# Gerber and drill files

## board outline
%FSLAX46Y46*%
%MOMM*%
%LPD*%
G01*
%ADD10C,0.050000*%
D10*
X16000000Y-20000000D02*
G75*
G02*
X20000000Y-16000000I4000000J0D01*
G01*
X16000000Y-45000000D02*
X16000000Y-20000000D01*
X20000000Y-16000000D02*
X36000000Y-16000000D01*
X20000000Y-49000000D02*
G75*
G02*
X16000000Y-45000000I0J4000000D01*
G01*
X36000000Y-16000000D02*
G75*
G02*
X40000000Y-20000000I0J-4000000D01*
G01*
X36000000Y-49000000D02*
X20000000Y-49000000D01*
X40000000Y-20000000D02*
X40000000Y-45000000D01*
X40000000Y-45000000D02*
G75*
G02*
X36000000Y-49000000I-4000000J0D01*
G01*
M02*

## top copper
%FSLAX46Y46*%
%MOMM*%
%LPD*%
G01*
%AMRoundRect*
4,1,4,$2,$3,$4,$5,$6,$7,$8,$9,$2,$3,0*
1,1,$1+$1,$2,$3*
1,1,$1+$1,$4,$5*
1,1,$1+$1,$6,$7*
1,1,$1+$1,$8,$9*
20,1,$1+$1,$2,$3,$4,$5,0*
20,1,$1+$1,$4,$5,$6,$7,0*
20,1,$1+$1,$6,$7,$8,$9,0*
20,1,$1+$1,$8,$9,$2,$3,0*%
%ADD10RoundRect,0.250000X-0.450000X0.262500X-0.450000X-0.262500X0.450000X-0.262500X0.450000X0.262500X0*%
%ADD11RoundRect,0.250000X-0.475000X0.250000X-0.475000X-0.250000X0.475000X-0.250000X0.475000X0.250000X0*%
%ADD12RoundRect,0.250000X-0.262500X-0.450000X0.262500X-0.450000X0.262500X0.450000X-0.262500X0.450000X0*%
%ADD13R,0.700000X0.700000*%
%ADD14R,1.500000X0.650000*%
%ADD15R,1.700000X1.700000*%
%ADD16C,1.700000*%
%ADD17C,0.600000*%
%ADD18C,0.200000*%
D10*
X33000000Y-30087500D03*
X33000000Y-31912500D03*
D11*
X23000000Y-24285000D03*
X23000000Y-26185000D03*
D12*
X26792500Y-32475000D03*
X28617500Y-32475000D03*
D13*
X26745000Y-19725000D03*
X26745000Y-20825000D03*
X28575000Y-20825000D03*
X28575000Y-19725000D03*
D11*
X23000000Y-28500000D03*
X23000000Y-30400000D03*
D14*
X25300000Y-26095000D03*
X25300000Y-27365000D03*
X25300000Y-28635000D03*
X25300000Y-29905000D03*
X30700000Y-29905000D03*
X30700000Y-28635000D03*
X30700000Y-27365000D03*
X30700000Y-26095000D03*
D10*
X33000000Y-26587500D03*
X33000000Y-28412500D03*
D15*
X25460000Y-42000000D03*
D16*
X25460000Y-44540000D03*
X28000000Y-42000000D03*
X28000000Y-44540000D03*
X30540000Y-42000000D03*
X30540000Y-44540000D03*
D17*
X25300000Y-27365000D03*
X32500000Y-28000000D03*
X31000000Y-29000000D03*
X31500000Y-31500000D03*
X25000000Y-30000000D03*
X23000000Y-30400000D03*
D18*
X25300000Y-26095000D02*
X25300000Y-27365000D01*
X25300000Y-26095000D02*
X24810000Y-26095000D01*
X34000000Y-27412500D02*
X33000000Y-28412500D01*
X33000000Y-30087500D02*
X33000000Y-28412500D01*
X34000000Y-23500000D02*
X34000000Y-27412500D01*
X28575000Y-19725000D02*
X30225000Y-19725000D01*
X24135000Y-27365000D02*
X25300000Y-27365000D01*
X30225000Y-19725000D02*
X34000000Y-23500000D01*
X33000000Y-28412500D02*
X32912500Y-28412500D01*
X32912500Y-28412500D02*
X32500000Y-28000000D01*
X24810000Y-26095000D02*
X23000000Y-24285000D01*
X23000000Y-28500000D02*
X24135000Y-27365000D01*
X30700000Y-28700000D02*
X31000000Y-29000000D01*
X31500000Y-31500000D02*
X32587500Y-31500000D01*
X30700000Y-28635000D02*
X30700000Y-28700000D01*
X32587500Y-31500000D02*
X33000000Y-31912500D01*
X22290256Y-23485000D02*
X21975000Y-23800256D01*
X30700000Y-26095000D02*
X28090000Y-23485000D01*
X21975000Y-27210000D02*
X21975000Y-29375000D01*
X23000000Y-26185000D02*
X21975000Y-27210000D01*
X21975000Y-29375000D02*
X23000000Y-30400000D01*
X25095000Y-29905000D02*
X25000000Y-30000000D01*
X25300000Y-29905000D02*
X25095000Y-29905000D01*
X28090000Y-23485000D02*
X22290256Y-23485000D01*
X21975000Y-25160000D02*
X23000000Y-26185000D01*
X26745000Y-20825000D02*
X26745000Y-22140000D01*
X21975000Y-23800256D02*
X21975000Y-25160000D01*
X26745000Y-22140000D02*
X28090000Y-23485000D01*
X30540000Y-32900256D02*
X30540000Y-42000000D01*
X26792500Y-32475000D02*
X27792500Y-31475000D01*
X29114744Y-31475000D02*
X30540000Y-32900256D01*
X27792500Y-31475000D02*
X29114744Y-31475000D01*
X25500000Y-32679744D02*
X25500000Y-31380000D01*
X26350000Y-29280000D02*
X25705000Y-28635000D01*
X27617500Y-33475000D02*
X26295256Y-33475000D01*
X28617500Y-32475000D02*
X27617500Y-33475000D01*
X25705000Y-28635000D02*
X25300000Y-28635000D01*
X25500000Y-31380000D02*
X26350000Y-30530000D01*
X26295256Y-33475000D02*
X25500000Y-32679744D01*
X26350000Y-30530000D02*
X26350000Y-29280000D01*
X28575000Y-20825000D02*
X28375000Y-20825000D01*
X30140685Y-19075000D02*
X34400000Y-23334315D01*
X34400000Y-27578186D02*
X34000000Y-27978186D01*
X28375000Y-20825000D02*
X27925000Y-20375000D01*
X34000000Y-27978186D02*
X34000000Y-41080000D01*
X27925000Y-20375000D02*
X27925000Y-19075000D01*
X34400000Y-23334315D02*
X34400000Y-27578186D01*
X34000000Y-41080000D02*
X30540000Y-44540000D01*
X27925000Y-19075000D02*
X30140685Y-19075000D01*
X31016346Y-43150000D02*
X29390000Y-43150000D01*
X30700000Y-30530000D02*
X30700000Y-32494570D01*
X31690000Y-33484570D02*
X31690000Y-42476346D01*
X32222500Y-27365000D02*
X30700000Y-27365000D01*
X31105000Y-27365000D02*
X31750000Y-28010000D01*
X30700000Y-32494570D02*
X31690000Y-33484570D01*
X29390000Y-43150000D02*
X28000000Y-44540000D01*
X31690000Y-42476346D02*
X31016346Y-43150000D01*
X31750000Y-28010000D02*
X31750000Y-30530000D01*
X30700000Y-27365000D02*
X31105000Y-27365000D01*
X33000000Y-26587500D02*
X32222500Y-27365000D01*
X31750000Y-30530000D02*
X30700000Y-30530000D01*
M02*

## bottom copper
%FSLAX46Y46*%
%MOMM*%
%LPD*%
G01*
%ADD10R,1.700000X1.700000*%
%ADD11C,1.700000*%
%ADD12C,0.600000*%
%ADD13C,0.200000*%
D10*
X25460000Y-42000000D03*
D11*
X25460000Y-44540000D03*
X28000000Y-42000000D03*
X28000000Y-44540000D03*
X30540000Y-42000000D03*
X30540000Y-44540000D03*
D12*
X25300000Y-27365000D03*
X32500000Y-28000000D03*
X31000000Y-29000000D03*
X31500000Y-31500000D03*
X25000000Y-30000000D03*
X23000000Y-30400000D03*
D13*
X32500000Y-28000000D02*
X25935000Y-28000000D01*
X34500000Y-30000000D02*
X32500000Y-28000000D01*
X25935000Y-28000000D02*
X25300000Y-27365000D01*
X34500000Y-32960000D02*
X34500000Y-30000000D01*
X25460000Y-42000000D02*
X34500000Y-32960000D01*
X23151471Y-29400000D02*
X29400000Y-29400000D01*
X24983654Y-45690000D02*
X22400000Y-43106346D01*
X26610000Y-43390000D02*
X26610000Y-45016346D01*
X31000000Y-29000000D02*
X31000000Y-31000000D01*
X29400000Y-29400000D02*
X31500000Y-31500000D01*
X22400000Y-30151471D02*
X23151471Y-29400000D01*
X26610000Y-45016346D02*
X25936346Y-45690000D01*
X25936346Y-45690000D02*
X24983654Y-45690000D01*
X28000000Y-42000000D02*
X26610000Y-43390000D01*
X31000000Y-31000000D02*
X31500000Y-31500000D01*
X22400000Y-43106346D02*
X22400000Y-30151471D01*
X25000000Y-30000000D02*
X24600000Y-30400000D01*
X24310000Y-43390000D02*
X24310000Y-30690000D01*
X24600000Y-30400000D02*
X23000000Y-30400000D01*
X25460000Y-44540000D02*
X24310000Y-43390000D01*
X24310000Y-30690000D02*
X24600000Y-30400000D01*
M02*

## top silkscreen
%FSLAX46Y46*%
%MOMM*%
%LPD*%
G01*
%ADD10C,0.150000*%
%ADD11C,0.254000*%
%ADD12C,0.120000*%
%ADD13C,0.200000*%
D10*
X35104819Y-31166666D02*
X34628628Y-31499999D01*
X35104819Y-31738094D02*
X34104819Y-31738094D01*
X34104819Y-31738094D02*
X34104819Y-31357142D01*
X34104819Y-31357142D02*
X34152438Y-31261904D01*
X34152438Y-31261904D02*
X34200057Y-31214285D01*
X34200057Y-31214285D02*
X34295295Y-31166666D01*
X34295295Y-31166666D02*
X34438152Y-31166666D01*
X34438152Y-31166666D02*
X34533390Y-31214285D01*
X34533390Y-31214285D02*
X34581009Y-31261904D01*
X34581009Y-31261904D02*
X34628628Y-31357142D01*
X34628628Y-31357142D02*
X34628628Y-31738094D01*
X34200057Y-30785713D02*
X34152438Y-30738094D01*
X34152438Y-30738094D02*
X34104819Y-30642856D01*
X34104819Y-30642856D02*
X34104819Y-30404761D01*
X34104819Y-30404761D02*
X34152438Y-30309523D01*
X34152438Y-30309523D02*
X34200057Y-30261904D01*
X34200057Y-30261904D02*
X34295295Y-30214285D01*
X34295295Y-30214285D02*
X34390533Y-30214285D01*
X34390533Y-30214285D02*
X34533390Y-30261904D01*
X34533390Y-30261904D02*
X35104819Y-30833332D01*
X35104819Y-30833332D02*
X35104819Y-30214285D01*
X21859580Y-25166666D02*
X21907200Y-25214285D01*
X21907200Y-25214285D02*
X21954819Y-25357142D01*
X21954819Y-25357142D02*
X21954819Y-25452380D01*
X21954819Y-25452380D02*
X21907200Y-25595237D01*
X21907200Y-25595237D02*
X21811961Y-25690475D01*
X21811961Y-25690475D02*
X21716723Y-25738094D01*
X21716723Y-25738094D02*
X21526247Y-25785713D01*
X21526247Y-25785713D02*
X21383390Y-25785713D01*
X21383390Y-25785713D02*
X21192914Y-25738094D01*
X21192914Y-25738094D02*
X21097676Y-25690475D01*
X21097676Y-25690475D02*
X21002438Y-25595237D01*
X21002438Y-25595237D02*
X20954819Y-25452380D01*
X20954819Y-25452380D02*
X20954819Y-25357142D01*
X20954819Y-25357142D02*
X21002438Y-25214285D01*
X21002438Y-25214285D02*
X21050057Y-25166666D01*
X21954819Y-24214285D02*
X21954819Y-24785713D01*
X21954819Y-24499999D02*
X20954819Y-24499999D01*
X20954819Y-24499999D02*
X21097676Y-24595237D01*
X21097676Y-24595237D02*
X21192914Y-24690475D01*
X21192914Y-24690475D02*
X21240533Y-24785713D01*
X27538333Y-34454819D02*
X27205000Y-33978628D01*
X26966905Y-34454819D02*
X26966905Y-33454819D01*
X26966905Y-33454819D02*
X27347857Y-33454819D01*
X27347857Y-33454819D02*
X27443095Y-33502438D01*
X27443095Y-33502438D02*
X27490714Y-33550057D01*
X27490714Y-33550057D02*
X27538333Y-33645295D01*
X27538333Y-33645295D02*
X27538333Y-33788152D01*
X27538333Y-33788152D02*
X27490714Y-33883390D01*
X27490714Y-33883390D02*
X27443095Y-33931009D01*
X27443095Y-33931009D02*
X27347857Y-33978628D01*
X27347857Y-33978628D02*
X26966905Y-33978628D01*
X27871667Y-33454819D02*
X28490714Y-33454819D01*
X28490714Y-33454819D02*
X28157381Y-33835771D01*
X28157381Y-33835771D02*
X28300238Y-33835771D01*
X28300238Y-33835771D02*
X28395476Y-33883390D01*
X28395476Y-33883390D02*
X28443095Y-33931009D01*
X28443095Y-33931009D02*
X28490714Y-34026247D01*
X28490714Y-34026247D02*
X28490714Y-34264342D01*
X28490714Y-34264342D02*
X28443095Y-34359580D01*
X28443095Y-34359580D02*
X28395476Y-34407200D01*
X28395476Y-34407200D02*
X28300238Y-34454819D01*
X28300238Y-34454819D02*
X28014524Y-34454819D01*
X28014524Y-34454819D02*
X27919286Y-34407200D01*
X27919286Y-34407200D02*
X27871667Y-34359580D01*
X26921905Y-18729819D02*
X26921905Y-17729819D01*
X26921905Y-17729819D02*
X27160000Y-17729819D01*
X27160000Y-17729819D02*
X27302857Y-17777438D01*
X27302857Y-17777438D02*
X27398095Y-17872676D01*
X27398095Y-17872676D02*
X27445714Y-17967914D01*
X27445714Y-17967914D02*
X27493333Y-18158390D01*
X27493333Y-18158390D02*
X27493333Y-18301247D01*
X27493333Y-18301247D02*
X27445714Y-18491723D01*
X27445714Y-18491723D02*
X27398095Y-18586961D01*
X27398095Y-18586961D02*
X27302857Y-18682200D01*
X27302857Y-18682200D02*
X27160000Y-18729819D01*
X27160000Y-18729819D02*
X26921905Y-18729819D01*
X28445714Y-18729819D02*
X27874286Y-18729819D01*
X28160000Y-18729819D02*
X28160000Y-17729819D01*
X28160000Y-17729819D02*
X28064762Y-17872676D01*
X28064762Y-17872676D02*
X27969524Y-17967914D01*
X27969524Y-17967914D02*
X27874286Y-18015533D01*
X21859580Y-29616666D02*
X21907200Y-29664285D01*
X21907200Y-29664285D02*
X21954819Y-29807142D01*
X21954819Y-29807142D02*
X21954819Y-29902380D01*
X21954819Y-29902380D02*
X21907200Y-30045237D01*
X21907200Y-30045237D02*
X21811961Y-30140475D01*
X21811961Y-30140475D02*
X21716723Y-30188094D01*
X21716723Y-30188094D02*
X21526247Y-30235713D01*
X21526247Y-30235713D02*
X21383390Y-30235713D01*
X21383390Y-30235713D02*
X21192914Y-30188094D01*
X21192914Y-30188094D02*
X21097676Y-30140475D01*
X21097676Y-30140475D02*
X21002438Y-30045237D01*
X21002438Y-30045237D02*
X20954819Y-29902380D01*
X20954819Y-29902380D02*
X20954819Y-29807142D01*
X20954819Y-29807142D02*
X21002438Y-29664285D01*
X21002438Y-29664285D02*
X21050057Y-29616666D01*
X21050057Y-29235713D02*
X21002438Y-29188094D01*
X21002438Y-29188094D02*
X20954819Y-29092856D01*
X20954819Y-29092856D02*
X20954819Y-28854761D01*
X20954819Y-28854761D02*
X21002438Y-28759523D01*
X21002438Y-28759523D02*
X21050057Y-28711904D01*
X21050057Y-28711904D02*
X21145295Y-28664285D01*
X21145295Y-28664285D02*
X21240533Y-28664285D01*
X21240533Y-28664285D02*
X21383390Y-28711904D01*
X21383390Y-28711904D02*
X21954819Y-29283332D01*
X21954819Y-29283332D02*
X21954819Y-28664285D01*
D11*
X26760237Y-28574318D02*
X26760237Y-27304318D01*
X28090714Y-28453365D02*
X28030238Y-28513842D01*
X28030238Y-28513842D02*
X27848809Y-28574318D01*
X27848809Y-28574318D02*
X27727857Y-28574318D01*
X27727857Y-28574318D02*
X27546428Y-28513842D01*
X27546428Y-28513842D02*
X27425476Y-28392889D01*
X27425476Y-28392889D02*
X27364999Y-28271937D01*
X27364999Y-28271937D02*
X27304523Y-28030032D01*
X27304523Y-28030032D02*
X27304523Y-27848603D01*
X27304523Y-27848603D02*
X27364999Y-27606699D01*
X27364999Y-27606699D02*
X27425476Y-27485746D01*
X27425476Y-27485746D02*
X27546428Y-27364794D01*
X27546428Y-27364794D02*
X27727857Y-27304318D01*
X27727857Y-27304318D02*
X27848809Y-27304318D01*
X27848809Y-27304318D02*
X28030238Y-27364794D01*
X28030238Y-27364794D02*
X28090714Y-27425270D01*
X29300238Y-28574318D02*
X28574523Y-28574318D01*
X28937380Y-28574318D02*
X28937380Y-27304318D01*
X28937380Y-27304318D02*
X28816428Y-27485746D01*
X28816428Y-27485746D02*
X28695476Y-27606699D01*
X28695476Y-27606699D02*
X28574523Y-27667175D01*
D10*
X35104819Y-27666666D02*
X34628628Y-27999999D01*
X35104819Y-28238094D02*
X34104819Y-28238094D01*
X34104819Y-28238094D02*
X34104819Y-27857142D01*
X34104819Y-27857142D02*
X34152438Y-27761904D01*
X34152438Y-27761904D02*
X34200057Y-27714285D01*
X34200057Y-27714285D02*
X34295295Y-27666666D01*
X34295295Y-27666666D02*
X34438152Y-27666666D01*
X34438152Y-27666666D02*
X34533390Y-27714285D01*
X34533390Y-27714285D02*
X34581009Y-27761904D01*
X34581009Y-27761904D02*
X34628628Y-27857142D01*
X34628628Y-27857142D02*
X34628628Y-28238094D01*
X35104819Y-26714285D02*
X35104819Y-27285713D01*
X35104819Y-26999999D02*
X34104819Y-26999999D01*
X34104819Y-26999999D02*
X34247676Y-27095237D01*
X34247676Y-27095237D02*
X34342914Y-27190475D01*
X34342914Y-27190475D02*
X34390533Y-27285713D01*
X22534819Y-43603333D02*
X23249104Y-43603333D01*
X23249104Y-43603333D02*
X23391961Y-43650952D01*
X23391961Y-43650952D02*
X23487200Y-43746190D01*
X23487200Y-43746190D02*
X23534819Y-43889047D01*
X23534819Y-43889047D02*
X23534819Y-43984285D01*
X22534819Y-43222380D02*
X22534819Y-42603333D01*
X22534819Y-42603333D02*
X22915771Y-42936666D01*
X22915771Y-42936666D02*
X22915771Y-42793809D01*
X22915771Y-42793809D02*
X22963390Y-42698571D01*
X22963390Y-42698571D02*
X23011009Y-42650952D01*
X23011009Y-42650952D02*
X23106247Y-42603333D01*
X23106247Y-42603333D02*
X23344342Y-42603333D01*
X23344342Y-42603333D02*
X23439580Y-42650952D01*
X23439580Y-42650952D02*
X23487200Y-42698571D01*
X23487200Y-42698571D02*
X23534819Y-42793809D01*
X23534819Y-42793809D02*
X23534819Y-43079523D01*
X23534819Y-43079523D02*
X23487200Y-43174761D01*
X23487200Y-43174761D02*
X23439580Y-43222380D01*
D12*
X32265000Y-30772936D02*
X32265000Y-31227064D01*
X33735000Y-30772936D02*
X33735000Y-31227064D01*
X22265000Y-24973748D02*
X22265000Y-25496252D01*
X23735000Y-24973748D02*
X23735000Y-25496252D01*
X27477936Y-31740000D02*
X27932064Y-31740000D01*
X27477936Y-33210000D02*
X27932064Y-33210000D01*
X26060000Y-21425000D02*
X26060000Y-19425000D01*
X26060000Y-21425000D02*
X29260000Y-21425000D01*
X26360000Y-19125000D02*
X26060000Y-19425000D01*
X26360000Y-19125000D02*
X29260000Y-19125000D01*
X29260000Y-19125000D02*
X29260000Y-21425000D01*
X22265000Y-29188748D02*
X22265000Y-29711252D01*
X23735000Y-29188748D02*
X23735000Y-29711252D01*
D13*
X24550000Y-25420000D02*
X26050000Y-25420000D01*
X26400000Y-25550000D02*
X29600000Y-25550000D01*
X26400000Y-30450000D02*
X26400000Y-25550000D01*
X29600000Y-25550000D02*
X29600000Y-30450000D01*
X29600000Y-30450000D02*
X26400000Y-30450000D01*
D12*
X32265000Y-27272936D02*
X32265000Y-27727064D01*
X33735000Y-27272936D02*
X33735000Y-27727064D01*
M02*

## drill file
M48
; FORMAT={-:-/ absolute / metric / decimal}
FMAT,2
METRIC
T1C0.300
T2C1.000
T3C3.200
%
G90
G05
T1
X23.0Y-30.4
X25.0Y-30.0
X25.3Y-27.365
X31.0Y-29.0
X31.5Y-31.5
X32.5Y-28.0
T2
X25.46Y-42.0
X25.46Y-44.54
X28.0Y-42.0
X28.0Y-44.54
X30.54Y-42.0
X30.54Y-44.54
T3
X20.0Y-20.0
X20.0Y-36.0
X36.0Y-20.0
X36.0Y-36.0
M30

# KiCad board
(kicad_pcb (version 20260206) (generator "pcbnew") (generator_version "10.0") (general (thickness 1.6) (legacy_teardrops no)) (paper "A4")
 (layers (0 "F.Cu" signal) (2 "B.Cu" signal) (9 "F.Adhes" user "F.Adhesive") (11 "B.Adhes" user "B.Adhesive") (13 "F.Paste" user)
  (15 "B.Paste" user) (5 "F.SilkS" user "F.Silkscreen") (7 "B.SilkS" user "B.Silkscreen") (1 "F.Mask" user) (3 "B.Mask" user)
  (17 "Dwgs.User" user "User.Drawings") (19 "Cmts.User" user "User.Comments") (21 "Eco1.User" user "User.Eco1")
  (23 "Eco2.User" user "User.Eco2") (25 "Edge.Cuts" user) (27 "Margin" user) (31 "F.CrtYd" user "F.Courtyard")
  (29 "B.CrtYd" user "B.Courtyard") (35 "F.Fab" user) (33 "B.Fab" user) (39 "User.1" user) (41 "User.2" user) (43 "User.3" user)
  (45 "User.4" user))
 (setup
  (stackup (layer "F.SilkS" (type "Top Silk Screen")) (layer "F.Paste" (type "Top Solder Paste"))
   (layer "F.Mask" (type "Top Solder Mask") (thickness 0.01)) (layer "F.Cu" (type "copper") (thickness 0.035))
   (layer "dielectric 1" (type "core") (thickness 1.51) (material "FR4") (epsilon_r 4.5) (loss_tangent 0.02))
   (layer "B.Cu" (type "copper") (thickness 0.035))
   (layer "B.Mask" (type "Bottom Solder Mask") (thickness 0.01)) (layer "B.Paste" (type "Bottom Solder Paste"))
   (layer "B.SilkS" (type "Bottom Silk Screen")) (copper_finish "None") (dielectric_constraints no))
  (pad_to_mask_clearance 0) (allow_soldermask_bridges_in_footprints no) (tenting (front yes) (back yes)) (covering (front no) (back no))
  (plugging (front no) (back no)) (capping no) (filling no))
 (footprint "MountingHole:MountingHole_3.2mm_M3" (layer "F.Cu") (at 36 20)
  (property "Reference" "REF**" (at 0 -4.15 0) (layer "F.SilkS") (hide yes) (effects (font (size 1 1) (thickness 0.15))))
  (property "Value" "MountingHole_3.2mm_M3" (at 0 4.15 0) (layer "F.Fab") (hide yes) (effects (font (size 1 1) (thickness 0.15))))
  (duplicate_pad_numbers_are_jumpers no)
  (pad "" np_thru_hole circle (at 0 0) (size 3.2 3.2) (drill 3.2) (layers "*.Cu" "*.Mask")))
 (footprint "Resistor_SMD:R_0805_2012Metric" (layer "F.Cu") (at 33 31 -90)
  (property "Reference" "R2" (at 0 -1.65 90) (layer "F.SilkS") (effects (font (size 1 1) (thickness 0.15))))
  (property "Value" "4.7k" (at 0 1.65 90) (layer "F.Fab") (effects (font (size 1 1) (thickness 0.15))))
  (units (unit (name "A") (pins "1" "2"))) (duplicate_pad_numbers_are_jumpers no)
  (fp_line (start -0.227064 0.735) (end 0.227064 0.735) (stroke (width 0.12) (type solid)) (layer "F.SilkS"))
  (fp_line (start -0.227064 -0.735) (end 0.227064 -0.735) (stroke (width 0.12) (type solid)) (layer "F.SilkS"))
  (pad "1" smd roundrect (at -0.9125 0 270) (size 1.025 1.4) (layers "F.Cu" "F.Mask" "F.Paste") (roundrect_rratio 0.243902) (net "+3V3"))
  (pad "2" smd roundrect (at 0.9125 0 270) (size 1.025 1.4) (layers "F.Cu" "F.Mask" "F.Paste") (roundrect_rratio 0.243902)
   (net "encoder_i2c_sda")))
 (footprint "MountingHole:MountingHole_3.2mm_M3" (layer "F.Cu") (at 36 36)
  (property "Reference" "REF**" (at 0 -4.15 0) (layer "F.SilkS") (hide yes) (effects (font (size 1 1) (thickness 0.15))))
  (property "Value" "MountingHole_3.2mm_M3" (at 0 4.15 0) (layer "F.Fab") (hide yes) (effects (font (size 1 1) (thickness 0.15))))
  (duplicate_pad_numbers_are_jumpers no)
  (pad "" np_thru_hole circle (at 0 0) (size 3.2 3.2) (drill 3.2) (layers "*.Cu" "*.Mask")))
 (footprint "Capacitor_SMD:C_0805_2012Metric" (layer "F.Cu") (at 23 25.235 -90)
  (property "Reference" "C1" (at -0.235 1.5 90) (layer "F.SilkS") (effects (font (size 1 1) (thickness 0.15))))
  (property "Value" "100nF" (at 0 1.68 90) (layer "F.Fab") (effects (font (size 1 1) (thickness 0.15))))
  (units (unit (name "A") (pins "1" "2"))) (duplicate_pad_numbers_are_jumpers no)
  (fp_line (start -0.261252 0.735) (end 0.261252 0.735) (stroke (width 0.12) (type solid)) (layer "F.SilkS"))
  (fp_line (start -0.261252 -0.735) (end 0.261252 -0.735) (stroke (width 0.12) (type solid)) (layer "F.SilkS"))
  (pad "1" smd roundrect (at -0.95 0 270) (size 1 1.45) (layers "F.Cu" "F.Mask" "F.Paste") (roundrect_rratio 0.25) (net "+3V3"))
  (pad "2" smd roundrect (at 0.95 0 270) (size 1 1.45) (layers "F.Cu" "F.Mask" "F.Paste") (roundrect_rratio 0.25) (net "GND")))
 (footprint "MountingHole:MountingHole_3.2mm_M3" (layer "F.Cu") (at 20 20)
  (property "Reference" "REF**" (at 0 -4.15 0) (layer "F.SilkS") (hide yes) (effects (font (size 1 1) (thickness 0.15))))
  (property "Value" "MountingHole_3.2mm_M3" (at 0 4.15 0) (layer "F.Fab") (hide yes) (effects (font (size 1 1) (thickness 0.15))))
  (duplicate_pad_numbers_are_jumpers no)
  (pad "" np_thru_hole circle (at 0 0) (size 3.2 3.2) (drill 3.2) (layers "*.Cu" "*.Mask")))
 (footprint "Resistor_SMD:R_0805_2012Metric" (layer "F.Cu") (at 27.705 32.475)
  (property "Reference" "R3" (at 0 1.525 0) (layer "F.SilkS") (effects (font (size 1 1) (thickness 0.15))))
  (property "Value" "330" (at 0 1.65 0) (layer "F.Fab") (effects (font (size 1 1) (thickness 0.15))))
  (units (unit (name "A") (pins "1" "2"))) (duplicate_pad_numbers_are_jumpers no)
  (fp_line (start -0.227064 -0.735) (end 0.227064 -0.735) (stroke (width 0.12) (type solid)) (layer "F.SilkS"))
  (fp_line (start -0.227064 0.735) (end 0.227064 0.735) (stroke (width 0.12) (type solid)) (layer "F.SilkS"))
  (pad "1" smd roundrect (at -0.9125 0) (size 1.025 1.4) (layers "F.Cu" "F.Mask" "F.Paste") (roundrect_rratio 0.243902)
   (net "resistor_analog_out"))
  (pad "2" smd roundrect (at 0.9125 0) (size 1.025 1.4) (layers "F.Cu" "F.Mask" "F.Paste") (roundrect_rratio 0.243902)
   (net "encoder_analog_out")))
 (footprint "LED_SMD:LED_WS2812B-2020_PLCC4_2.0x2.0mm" (layer "F.Cu") (at 27.66 20.275)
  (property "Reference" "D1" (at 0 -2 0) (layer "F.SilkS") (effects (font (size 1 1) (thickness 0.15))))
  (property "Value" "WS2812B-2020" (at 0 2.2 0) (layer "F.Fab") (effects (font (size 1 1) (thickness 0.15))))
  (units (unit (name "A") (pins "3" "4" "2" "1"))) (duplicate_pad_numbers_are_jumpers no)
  (fp_line (start -1.6 1.15) (end -1.6 -0.85) (stroke (width 0.12) (type solid)) (layer "F.SilkS"))
  (fp_line (start -1.6 1.15) (end 1.6 1.15) (stroke (width 0.12) (type solid)) (layer "F.SilkS"))
  (fp_line (start -1.3 -1.15) (end -1.6 -0.85) (stroke (width 0.12) (type default)) (layer "F.SilkS"))
  (fp_line (start -1.3 -1.15) (end 1.6 -1.15) (stroke (width 0.12) (type solid)) (layer "F.SilkS"))
  (fp_line (start 1.6 -1.15) (end 1.6 1.15) (stroke (width 0.12) (type solid)) (layer "F.SilkS"))
  (pad "1" smd rect (at -0.915 -0.55) (size 0.7 0.7) (layers "F.Cu" "F.Mask" "F.Paste") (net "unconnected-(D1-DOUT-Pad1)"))
  (pad "2" smd rect (at -0.915 0.55) (size 0.7 0.7) (layers "F.Cu" "F.Mask" "F.Paste") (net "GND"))
  (pad "3" smd rect (at 0.915 0.55) (size 0.7 0.7) (layers "F.Cu" "F.Mask" "F.Paste") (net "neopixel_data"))
  (pad "4" smd rect (at 0.915 -0.55) (size 0.7 0.7) (layers "F.Cu" "F.Mask" "F.Paste") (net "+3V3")))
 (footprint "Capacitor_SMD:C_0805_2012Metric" (layer "F.Cu") (at 23 29.45 -90)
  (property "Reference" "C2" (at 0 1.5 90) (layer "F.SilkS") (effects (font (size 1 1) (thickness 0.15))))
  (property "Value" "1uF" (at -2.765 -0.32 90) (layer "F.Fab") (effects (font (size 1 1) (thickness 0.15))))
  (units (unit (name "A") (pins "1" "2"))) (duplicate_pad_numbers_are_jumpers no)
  (fp_line (start -0.261252 0.735) (end 0.261252 0.735) (stroke (width 0.12) (type solid)) (layer "F.SilkS"))
  (fp_line (start -0.261252 -0.735) (end 0.261252 -0.735) (stroke (width 0.12) (type solid)) (layer "F.SilkS"))
  (pad "1" smd roundrect (at -0.95 0 270) (size 1 1.45) (layers "F.Cu" "F.Mask" "F.Paste") (roundrect_rratio 0.25) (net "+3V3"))
  (pad "2" smd roundrect (at 0.95 0 270) (size 1 1.45) (layers "F.Cu" "F.Mask" "F.Paste") (roundrect_rratio 0.25) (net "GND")))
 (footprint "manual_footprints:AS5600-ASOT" (layer "F.Cu") (at 28 28)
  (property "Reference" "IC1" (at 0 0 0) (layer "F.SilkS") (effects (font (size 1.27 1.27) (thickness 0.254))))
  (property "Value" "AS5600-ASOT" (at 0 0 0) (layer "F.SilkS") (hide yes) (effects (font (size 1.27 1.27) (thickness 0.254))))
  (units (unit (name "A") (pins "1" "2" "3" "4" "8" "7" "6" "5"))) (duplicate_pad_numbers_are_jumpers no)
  (fp_line (start -3.45 -2.58) (end -1.95 -2.58) (stroke (width 0.2) (type solid)) (layer "F.SilkS"))
  (fp_line (start -1.6 -2.45) (end 1.6 -2.45) (stroke (width 0.2) (type solid)) (layer "F.SilkS"))
  (fp_line (start -1.6 2.45) (end -1.6 -2.45) (stroke (width 0.2) (type solid)) (layer "F.SilkS"))
  (fp_line (start 1.6 -2.45) (end 1.6 2.45) (stroke (width 0.2) (type solid)) (layer "F.SilkS"))
  (fp_line (start 1.6 2.45) (end -1.6 2.45) (stroke (width 0.2) (type solid)) (layer "F.SilkS"))
  (pad "1" smd rect (at -2.7 -1.905 90) (size 0.65 1.5) (layers "F.Cu" "F.Mask" "F.Paste") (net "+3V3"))
  (pad "2" smd rect (at -2.7 -0.635 90) (size 0.65 1.5) (layers "F.Cu" "F.Mask" "F.Paste") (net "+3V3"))
  (pad "3" smd rect (at -2.7 0.635 90) (size 0.65 1.5) (layers "F.Cu" "F.Mask" "F.Paste") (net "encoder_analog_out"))
  (pad "4" smd rect (at -2.7 1.905 90) (size 0.65 1.5) (layers "F.Cu" "F.Mask" "F.Paste") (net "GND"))
  (pad "5" smd rect (at 2.7 1.905 90) (size 0.65 1.5) (layers "F.Cu" "F.Mask" "F.Paste") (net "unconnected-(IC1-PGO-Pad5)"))
  (pad "6" smd rect (at 2.7 0.635 90) (size 0.65 1.5) (layers "F.Cu" "F.Mask" "F.Paste") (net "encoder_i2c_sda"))
  (pad "7" smd rect (at 2.7 -0.635 90) (size 0.65 1.5) (layers "F.Cu" "F.Mask" "F.Paste") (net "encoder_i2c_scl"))
  (pad "8" smd rect (at 2.7 -1.905 90) (size 0.65 1.5) (layers "F.Cu" "F.Mask" "F.Paste") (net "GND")))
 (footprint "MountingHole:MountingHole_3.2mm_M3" (layer "F.Cu") (at 20 36)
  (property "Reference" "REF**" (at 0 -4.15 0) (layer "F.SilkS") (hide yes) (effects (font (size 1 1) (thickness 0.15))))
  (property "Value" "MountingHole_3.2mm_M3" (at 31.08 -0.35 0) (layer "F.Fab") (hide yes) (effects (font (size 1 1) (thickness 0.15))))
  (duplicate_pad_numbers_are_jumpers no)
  (pad "" np_thru_hole circle (at 0 0) (size 3.2 3.2) (drill 3.2) (layers "*.Cu" "*.Mask")))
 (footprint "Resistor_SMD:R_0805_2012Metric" (layer "F.Cu") (at 33 27.5 -90)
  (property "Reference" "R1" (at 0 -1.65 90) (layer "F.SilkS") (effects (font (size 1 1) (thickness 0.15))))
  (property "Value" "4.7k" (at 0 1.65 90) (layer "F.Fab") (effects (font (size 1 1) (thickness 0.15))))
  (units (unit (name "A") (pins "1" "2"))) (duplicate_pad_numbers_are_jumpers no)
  (fp_line (start -0.227064 0.735) (end 0.227064 0.735) (stroke (width 0.12) (type solid)) (layer "F.SilkS"))
  (fp_line (start -0.227064 -0.735) (end 0.227064 -0.735) (stroke (width 0.12) (type solid)) (layer "F.SilkS"))
  (pad "1" smd roundrect (at -0.9125 0 270) (size 1.025 1.4) (layers "F.Cu" "F.Mask" "F.Paste") (roundrect_rratio 0.243902)
   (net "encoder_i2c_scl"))
  (pad "2" smd roundrect (at 0.9125 0 270) (size 1.025 1.4) (layers "F.Cu" "F.Mask" "F.Paste") (roundrect_rratio 0.243902) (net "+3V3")))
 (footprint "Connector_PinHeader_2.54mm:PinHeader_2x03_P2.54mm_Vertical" (layer "B.Cu") (at 25.46 42 -90)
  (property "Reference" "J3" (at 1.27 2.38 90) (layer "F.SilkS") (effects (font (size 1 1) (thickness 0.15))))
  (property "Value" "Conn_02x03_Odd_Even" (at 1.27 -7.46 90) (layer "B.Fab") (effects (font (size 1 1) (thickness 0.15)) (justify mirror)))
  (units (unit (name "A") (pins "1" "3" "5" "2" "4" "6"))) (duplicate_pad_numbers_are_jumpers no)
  (pad "1" thru_hole rect (at 0 0 270) (size 1.7 1.7) (drill 1) (layers "*.Cu" "*.Mask") (remove_unused_layers no) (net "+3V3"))
  (pad "2" thru_hole circle (at 2.54 0 270) (size 1.7 1.7) (drill 1) (layers "*.Cu" "*.Mask") (remove_unused_layers no) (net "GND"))
  (pad "3" thru_hole circle (at 0 -2.54 270) (size 1.7 1.7) (drill 1) (layers "*.Cu" "*.Mask") (remove_unused_layers no)
   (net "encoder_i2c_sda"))
  (pad "4" thru_hole circle (at 2.54 -2.54 270) (size 1.7 1.7) (drill 1) (layers "*.Cu" "*.Mask") (remove_unused_layers no)
   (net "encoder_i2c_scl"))
  (pad "5" thru_hole circle (at 0 -5.08 270) (size 1.7 1.7) (drill 1) (layers "*.Cu" "*.Mask") (remove_unused_layers no)
   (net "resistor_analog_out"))
  (pad "6" thru_hole circle (at 2.54 -5.08 270) (size 1.7 1.7) (drill 1) (layers "*.Cu" "*.Mask") (remove_unused_layers no)
   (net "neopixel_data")))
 (gr_arc (start 16 20) (mid 17.171573 17.171573) (end 20 16) (stroke (width 0.05) (type solid)) (layer "Edge.Cuts"))
 (gr_line (start 16 45) (end 16 20) (stroke (width 0.05) (type solid)) (layer "Edge.Cuts"))
 (gr_line (start 20 16) (end 36 16) (stroke (width 0.05) (type solid)) (layer "Edge.Cuts"))
 (gr_arc (start 20 49) (mid 17.171573 47.828427) (end 16 45) (stroke (width 0.05) (type solid)) (layer "Edge.Cuts"))
 (gr_arc (start 36 16) (mid 38.828427 17.171573) (end 40 20) (stroke (width 0.05) (type solid)) (layer "Edge.Cuts"))
 (gr_line (start 36 49) (end 20 49) (stroke (width 0.05) (type solid)) (layer "Edge.Cuts"))
 (gr_line (start 40 20) (end 40 45) (stroke (width 0.05) (type solid)) (layer "Edge.Cuts"))
 (gr_arc (start 40 45) (mid 38.828427 47.828427) (end 36 49) (stroke (width 0.05) (type solid)) (layer "Edge.Cuts"))
 (segment (start 25.3 26.095) (end 25.3 27.365) (width 0.2) (layer "F.Cu") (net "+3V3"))
 (segment (start 25.3 26.095) (end 24.81 26.095) (width 0.2) (layer "F.Cu") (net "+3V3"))
 (segment (start 34 27.4125) (end 33 28.4125) (width 0.2) (layer "F.Cu") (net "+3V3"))
 (segment (start 33 30.0875) (end 33 28.4125) (width 0.2) (layer "F.Cu") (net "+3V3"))
 (segment (start 34 23.5) (end 34 27.4125) (width 0.2) (layer "F.Cu") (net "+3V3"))
 (segment (start 28.575 19.725) (end 30.225 19.725) (width 0.2) (layer "F.Cu") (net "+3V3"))
 (segment (start 24.135 27.365) (end 25.3 27.365) (width 0.2) (layer "F.Cu") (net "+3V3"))
 (segment (start 30.225 19.725) (end 34 23.5) (width 0.2) (layer "F.Cu") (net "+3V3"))
 (segment (start 33 28.4125) (end 32.9125 28.4125) (width 0.2) (layer "F.Cu") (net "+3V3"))
 (segment (start 32.9125 28.4125) (end 32.5 28) (width 0.2) (layer "F.Cu") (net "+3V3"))
 (segment (start 24.81 26.095) (end 23 24.285) (width 0.2) (layer "F.Cu") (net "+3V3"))
 (segment (start 23 28.5) (end 24.135 27.365) (width 0.2) (layer "F.Cu") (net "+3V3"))
 (via (at 25.3 27.365) (size 0.6) (drill 0.3) (layers "F.Cu" "B.Cu") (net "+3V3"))
 (via (at 32.5 28) (size 0.6) (drill 0.3) (layers "F.Cu" "B.Cu") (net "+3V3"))
 (segment (start 32.5 28) (end 25.935 28) (width 0.2) (layer "B.Cu") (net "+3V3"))
 (segment (start 34.5 30) (end 32.5 28) (width 0.2) (layer "B.Cu") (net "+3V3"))
 (segment (start 25.935 28) (end 25.3 27.365) (width 0.2) (layer "B.Cu") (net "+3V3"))
 (segment (start 34.5 32.96) (end 34.5 30) (width 0.2) (layer "B.Cu") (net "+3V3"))
 (segment (start 25.46 42) (end 34.5 32.96) (width 0.2) (layer "B.Cu") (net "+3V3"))
 (segment (start 30.7 28.7) (end 31 29) (width 0.2) (layer "F.Cu") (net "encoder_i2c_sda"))
 (segment (start 31.5 31.5) (end 32.5875 31.5) (width 0.2) (layer "F.Cu") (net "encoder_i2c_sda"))
 (segment (start 30.7 28.635) (end 30.7 28.7) (width 0.2) (layer "F.Cu") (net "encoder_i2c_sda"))
 (segment (start 32.5875 31.5) (end 33 31.9125) (width 0.2) (layer "F.Cu") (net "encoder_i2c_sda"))
 (via (at 31 29) (size 0.6) (drill 0.3) (layers "F.Cu" "B.Cu") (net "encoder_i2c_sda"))
 (via (at 31.5 31.5) (size 0.6) (drill 0.3) (layers "F.Cu" "B.Cu") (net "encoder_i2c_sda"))
 (segment (start 23.151471 29.4) (end 29.4 29.4) (width 0.2) (layer "B.Cu") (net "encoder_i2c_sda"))
 (segment (start 24.983654 45.69) (end 22.4 43.106346) (width 0.2) (layer "B.Cu") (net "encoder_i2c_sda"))
 (segment (start 26.61 43.39) (end 26.61 45.016346) (width 0.2) (layer "B.Cu") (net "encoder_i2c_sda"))
 (segment (start 31 29) (end 31 31) (width 0.2) (layer "B.Cu") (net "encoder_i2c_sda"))
 (segment (start 29.4 29.4) (end 31.5 31.5) (width 0.2) (layer "B.Cu") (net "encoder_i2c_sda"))
 (segment (start 22.4 30.151471) (end 23.151471 29.4) (width 0.2) (layer "B.Cu") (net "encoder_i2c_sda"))
 (segment (start 26.61 45.016346) (end 25.936346 45.69) (width 0.2) (layer "B.Cu") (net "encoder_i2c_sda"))
 (segment (start 25.936346 45.69) (end 24.983654 45.69) (width 0.2) (layer "B.Cu") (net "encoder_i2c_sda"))
 (segment (start 28 42) (end 26.61 43.39) (width 0.2) (layer "B.Cu") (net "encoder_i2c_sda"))
 (segment (start 31 31) (end 31.5 31.5) (width 0.2) (layer "B.Cu") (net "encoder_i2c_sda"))
 (segment (start 22.4 43.106346) (end 22.4 30.151471) (width 0.2) (layer "B.Cu") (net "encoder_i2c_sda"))
 (segment (start 22.290256 23.485) (end 21.975 23.800256) (width 0.2) (layer "F.Cu") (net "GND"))
 (segment (start 30.7 26.095) (end 28.09 23.485) (width 0.2) (layer "F.Cu") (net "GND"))
 (segment (start 21.975 27.21) (end 21.975 29.375) (width 0.2) (layer "F.Cu") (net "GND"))
 (segment (start 23 26.185) (end 21.975 27.21) (width 0.2) (layer "F.Cu") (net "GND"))
 (segment (start 21.975 29.375) (end 23 30.4) (width 0.2) (layer "F.Cu") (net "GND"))
 (segment (start 25.095 29.905) (end 25 30) (width 0.2) (layer "F.Cu") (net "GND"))
 (segment (start 25.3 29.905) (end 25.095 29.905) (width 0.2) (layer "F.Cu") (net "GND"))
 (segment (start 28.09 23.485) (end 22.290256 23.485) (width 0.2) (layer "F.Cu") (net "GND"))
 (segment (start 21.975 25.16) (end 23 26.185) (width 0.2) (layer "F.Cu") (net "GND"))
 (segment (start 26.745 20.825) (end 26.745 22.14) (width 0.2) (layer "F.Cu") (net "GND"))
 (segment (start 21.975 23.800256) (end 21.975 25.16) (width 0.2) (layer "F.Cu") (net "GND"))
 (segment (start 26.745 22.14) (end 28.09 23.485) (width 0.2) (layer "F.Cu") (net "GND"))
 (via (at 25 30) (size 0.6) (drill 0.3) (layers "F.Cu" "B.Cu") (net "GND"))
 (via (at 23 30.4) (size 0.6) (drill 0.3) (layers "F.Cu" "B.Cu") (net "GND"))
 (segment (start 25 30) (end 24.6 30.4) (width 0.2) (layer "B.Cu") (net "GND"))
 (segment (start 24.31 43.39) (end 24.31 30.69) (width 0.2) (layer "B.Cu") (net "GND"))
 (segment (start 24.6 30.4) (end 23 30.4) (width 0.2) (layer "B.Cu") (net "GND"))
 (segment (start 25.46 44.54) (end 24.31 43.39) (width 0.2) (layer "B.Cu") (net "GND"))
 (segment (start 24.31 30.69) (end 24.6 30.4) (width 0.2) (layer "B.Cu") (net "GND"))
 (segment (start 30.54 32.900256) (end 30.54 42) (width 0.2) (layer "F.Cu") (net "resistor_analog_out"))
 (segment (start 26.7925 32.475) (end 27.7925 31.475) (width 0.2) (layer "F.Cu") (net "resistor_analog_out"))
 (segment (start 29.114744 31.475) (end 30.54 32.900256) (width 0.2) (layer "F.Cu") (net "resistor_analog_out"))
 (segment (start 27.7925 31.475) (end 29.114744 31.475) (width 0.2) (layer "F.Cu") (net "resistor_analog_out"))
 (segment (start 25.5 32.679744) (end 25.5 31.38) (width 0.2) (layer "F.Cu") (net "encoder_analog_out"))
 (segment (start 26.35 29.28) (end 25.705 28.635) (width 0.2) (layer "F.Cu") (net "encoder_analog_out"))
 (segment (start 27.6175 33.475) (end 26.295256 33.475) (width 0.2) (layer "F.Cu") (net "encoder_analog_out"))
 (segment (start 28.6175 32.475) (end 27.6175 33.475) (width 0.2) (layer "F.Cu") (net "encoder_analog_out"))
 (segment (start 25.705 28.635) (end 25.3 28.635) (width 0.2) (layer "F.Cu") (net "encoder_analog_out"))
 (segment (start 25.5 31.38) (end 26.35 30.53) (width 0.2) (layer "F.Cu") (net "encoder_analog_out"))
 (segment (start 26.295256 33.475) (end 25.5 32.679744) (width 0.2) (layer "F.Cu") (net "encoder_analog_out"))
 (segment (start 26.35 30.53) (end 26.35 29.28) (width 0.2) (layer "F.Cu") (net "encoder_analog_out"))
 (segment (start 28.575 20.825) (end 28.375 20.825) (width 0.2) (layer "F.Cu") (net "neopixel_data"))
 (segment (start 30.140685 19.075) (end 34.4 23.334315) (width 0.2) (layer "F.Cu") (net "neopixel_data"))
 (segment (start 34.4 27.578186) (end 34 27.978186) (width 0.2) (layer "F.Cu") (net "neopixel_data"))
 (segment (start 28.375 20.825) (end 27.925 20.375) (width 0.2) (layer "F.Cu") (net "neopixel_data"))
 (segment (start 34 27.978186) (end 34 41.08) (width 0.2) (layer "F.Cu") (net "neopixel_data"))
 (segment (start 27.925 20.375) (end 27.925 19.075) (width 0.2) (layer "F.Cu") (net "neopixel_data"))
 (segment (start 34.4 23.334315) (end 34.4 27.578186) (width 0.2) (layer "F.Cu") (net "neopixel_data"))
 (segment (start 34 41.08) (end 30.54 44.54) (width 0.2) (layer "F.Cu") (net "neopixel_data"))
 (segment (start 27.925 19.075) (end 30.140685 19.075) (width 0.2) (layer "F.Cu") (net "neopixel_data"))
 (segment (start 31.016346 43.15) (end 29.39 43.15) (width 0.2) (layer "F.Cu") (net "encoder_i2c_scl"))
 (segment (start 30.7 30.53) (end 30.7 32.49457) (width 0.2) (layer "F.Cu") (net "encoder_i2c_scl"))
 (segment (start 31.69 33.48457) (end 31.69 42.476346) (width 0.2) (layer "F.Cu") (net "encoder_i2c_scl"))
 (segment (start 32.2225 27.365) (end 30.7 27.365) (width 0.2) (layer "F.Cu") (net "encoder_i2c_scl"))
 (segment (start 31.105 27.365) (end 31.75 28.01) (width 0.2) (layer "F.Cu") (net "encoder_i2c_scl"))
 (segment (start 30.7 32.49457) (end 31.69 33.48457) (width 0.2) (layer "F.Cu") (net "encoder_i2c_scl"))
 (segment (start 29.39 43.15) (end 28 44.54) (width 0.2) (layer "F.Cu") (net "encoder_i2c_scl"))
 (segment (start 31.69 42.476346) (end 31.016346 43.15) (width 0.2) (layer "F.Cu") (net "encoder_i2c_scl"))
 (segment (start 31.75 28.01) (end 31.75 30.53) (width 0.2) (layer "F.Cu") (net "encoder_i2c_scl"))
 (segment (start 30.7 27.365) (end 31.105 27.365) (width 0.2) (layer "F.Cu") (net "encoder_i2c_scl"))
 (segment (start 33 26.5875) (end 32.2225 27.365) (width 0.2) (layer "F.Cu") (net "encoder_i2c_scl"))
 (segment (start 31.75 30.53) (end 30.7 30.53) (width 0.2) (layer "F.Cu") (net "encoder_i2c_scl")))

